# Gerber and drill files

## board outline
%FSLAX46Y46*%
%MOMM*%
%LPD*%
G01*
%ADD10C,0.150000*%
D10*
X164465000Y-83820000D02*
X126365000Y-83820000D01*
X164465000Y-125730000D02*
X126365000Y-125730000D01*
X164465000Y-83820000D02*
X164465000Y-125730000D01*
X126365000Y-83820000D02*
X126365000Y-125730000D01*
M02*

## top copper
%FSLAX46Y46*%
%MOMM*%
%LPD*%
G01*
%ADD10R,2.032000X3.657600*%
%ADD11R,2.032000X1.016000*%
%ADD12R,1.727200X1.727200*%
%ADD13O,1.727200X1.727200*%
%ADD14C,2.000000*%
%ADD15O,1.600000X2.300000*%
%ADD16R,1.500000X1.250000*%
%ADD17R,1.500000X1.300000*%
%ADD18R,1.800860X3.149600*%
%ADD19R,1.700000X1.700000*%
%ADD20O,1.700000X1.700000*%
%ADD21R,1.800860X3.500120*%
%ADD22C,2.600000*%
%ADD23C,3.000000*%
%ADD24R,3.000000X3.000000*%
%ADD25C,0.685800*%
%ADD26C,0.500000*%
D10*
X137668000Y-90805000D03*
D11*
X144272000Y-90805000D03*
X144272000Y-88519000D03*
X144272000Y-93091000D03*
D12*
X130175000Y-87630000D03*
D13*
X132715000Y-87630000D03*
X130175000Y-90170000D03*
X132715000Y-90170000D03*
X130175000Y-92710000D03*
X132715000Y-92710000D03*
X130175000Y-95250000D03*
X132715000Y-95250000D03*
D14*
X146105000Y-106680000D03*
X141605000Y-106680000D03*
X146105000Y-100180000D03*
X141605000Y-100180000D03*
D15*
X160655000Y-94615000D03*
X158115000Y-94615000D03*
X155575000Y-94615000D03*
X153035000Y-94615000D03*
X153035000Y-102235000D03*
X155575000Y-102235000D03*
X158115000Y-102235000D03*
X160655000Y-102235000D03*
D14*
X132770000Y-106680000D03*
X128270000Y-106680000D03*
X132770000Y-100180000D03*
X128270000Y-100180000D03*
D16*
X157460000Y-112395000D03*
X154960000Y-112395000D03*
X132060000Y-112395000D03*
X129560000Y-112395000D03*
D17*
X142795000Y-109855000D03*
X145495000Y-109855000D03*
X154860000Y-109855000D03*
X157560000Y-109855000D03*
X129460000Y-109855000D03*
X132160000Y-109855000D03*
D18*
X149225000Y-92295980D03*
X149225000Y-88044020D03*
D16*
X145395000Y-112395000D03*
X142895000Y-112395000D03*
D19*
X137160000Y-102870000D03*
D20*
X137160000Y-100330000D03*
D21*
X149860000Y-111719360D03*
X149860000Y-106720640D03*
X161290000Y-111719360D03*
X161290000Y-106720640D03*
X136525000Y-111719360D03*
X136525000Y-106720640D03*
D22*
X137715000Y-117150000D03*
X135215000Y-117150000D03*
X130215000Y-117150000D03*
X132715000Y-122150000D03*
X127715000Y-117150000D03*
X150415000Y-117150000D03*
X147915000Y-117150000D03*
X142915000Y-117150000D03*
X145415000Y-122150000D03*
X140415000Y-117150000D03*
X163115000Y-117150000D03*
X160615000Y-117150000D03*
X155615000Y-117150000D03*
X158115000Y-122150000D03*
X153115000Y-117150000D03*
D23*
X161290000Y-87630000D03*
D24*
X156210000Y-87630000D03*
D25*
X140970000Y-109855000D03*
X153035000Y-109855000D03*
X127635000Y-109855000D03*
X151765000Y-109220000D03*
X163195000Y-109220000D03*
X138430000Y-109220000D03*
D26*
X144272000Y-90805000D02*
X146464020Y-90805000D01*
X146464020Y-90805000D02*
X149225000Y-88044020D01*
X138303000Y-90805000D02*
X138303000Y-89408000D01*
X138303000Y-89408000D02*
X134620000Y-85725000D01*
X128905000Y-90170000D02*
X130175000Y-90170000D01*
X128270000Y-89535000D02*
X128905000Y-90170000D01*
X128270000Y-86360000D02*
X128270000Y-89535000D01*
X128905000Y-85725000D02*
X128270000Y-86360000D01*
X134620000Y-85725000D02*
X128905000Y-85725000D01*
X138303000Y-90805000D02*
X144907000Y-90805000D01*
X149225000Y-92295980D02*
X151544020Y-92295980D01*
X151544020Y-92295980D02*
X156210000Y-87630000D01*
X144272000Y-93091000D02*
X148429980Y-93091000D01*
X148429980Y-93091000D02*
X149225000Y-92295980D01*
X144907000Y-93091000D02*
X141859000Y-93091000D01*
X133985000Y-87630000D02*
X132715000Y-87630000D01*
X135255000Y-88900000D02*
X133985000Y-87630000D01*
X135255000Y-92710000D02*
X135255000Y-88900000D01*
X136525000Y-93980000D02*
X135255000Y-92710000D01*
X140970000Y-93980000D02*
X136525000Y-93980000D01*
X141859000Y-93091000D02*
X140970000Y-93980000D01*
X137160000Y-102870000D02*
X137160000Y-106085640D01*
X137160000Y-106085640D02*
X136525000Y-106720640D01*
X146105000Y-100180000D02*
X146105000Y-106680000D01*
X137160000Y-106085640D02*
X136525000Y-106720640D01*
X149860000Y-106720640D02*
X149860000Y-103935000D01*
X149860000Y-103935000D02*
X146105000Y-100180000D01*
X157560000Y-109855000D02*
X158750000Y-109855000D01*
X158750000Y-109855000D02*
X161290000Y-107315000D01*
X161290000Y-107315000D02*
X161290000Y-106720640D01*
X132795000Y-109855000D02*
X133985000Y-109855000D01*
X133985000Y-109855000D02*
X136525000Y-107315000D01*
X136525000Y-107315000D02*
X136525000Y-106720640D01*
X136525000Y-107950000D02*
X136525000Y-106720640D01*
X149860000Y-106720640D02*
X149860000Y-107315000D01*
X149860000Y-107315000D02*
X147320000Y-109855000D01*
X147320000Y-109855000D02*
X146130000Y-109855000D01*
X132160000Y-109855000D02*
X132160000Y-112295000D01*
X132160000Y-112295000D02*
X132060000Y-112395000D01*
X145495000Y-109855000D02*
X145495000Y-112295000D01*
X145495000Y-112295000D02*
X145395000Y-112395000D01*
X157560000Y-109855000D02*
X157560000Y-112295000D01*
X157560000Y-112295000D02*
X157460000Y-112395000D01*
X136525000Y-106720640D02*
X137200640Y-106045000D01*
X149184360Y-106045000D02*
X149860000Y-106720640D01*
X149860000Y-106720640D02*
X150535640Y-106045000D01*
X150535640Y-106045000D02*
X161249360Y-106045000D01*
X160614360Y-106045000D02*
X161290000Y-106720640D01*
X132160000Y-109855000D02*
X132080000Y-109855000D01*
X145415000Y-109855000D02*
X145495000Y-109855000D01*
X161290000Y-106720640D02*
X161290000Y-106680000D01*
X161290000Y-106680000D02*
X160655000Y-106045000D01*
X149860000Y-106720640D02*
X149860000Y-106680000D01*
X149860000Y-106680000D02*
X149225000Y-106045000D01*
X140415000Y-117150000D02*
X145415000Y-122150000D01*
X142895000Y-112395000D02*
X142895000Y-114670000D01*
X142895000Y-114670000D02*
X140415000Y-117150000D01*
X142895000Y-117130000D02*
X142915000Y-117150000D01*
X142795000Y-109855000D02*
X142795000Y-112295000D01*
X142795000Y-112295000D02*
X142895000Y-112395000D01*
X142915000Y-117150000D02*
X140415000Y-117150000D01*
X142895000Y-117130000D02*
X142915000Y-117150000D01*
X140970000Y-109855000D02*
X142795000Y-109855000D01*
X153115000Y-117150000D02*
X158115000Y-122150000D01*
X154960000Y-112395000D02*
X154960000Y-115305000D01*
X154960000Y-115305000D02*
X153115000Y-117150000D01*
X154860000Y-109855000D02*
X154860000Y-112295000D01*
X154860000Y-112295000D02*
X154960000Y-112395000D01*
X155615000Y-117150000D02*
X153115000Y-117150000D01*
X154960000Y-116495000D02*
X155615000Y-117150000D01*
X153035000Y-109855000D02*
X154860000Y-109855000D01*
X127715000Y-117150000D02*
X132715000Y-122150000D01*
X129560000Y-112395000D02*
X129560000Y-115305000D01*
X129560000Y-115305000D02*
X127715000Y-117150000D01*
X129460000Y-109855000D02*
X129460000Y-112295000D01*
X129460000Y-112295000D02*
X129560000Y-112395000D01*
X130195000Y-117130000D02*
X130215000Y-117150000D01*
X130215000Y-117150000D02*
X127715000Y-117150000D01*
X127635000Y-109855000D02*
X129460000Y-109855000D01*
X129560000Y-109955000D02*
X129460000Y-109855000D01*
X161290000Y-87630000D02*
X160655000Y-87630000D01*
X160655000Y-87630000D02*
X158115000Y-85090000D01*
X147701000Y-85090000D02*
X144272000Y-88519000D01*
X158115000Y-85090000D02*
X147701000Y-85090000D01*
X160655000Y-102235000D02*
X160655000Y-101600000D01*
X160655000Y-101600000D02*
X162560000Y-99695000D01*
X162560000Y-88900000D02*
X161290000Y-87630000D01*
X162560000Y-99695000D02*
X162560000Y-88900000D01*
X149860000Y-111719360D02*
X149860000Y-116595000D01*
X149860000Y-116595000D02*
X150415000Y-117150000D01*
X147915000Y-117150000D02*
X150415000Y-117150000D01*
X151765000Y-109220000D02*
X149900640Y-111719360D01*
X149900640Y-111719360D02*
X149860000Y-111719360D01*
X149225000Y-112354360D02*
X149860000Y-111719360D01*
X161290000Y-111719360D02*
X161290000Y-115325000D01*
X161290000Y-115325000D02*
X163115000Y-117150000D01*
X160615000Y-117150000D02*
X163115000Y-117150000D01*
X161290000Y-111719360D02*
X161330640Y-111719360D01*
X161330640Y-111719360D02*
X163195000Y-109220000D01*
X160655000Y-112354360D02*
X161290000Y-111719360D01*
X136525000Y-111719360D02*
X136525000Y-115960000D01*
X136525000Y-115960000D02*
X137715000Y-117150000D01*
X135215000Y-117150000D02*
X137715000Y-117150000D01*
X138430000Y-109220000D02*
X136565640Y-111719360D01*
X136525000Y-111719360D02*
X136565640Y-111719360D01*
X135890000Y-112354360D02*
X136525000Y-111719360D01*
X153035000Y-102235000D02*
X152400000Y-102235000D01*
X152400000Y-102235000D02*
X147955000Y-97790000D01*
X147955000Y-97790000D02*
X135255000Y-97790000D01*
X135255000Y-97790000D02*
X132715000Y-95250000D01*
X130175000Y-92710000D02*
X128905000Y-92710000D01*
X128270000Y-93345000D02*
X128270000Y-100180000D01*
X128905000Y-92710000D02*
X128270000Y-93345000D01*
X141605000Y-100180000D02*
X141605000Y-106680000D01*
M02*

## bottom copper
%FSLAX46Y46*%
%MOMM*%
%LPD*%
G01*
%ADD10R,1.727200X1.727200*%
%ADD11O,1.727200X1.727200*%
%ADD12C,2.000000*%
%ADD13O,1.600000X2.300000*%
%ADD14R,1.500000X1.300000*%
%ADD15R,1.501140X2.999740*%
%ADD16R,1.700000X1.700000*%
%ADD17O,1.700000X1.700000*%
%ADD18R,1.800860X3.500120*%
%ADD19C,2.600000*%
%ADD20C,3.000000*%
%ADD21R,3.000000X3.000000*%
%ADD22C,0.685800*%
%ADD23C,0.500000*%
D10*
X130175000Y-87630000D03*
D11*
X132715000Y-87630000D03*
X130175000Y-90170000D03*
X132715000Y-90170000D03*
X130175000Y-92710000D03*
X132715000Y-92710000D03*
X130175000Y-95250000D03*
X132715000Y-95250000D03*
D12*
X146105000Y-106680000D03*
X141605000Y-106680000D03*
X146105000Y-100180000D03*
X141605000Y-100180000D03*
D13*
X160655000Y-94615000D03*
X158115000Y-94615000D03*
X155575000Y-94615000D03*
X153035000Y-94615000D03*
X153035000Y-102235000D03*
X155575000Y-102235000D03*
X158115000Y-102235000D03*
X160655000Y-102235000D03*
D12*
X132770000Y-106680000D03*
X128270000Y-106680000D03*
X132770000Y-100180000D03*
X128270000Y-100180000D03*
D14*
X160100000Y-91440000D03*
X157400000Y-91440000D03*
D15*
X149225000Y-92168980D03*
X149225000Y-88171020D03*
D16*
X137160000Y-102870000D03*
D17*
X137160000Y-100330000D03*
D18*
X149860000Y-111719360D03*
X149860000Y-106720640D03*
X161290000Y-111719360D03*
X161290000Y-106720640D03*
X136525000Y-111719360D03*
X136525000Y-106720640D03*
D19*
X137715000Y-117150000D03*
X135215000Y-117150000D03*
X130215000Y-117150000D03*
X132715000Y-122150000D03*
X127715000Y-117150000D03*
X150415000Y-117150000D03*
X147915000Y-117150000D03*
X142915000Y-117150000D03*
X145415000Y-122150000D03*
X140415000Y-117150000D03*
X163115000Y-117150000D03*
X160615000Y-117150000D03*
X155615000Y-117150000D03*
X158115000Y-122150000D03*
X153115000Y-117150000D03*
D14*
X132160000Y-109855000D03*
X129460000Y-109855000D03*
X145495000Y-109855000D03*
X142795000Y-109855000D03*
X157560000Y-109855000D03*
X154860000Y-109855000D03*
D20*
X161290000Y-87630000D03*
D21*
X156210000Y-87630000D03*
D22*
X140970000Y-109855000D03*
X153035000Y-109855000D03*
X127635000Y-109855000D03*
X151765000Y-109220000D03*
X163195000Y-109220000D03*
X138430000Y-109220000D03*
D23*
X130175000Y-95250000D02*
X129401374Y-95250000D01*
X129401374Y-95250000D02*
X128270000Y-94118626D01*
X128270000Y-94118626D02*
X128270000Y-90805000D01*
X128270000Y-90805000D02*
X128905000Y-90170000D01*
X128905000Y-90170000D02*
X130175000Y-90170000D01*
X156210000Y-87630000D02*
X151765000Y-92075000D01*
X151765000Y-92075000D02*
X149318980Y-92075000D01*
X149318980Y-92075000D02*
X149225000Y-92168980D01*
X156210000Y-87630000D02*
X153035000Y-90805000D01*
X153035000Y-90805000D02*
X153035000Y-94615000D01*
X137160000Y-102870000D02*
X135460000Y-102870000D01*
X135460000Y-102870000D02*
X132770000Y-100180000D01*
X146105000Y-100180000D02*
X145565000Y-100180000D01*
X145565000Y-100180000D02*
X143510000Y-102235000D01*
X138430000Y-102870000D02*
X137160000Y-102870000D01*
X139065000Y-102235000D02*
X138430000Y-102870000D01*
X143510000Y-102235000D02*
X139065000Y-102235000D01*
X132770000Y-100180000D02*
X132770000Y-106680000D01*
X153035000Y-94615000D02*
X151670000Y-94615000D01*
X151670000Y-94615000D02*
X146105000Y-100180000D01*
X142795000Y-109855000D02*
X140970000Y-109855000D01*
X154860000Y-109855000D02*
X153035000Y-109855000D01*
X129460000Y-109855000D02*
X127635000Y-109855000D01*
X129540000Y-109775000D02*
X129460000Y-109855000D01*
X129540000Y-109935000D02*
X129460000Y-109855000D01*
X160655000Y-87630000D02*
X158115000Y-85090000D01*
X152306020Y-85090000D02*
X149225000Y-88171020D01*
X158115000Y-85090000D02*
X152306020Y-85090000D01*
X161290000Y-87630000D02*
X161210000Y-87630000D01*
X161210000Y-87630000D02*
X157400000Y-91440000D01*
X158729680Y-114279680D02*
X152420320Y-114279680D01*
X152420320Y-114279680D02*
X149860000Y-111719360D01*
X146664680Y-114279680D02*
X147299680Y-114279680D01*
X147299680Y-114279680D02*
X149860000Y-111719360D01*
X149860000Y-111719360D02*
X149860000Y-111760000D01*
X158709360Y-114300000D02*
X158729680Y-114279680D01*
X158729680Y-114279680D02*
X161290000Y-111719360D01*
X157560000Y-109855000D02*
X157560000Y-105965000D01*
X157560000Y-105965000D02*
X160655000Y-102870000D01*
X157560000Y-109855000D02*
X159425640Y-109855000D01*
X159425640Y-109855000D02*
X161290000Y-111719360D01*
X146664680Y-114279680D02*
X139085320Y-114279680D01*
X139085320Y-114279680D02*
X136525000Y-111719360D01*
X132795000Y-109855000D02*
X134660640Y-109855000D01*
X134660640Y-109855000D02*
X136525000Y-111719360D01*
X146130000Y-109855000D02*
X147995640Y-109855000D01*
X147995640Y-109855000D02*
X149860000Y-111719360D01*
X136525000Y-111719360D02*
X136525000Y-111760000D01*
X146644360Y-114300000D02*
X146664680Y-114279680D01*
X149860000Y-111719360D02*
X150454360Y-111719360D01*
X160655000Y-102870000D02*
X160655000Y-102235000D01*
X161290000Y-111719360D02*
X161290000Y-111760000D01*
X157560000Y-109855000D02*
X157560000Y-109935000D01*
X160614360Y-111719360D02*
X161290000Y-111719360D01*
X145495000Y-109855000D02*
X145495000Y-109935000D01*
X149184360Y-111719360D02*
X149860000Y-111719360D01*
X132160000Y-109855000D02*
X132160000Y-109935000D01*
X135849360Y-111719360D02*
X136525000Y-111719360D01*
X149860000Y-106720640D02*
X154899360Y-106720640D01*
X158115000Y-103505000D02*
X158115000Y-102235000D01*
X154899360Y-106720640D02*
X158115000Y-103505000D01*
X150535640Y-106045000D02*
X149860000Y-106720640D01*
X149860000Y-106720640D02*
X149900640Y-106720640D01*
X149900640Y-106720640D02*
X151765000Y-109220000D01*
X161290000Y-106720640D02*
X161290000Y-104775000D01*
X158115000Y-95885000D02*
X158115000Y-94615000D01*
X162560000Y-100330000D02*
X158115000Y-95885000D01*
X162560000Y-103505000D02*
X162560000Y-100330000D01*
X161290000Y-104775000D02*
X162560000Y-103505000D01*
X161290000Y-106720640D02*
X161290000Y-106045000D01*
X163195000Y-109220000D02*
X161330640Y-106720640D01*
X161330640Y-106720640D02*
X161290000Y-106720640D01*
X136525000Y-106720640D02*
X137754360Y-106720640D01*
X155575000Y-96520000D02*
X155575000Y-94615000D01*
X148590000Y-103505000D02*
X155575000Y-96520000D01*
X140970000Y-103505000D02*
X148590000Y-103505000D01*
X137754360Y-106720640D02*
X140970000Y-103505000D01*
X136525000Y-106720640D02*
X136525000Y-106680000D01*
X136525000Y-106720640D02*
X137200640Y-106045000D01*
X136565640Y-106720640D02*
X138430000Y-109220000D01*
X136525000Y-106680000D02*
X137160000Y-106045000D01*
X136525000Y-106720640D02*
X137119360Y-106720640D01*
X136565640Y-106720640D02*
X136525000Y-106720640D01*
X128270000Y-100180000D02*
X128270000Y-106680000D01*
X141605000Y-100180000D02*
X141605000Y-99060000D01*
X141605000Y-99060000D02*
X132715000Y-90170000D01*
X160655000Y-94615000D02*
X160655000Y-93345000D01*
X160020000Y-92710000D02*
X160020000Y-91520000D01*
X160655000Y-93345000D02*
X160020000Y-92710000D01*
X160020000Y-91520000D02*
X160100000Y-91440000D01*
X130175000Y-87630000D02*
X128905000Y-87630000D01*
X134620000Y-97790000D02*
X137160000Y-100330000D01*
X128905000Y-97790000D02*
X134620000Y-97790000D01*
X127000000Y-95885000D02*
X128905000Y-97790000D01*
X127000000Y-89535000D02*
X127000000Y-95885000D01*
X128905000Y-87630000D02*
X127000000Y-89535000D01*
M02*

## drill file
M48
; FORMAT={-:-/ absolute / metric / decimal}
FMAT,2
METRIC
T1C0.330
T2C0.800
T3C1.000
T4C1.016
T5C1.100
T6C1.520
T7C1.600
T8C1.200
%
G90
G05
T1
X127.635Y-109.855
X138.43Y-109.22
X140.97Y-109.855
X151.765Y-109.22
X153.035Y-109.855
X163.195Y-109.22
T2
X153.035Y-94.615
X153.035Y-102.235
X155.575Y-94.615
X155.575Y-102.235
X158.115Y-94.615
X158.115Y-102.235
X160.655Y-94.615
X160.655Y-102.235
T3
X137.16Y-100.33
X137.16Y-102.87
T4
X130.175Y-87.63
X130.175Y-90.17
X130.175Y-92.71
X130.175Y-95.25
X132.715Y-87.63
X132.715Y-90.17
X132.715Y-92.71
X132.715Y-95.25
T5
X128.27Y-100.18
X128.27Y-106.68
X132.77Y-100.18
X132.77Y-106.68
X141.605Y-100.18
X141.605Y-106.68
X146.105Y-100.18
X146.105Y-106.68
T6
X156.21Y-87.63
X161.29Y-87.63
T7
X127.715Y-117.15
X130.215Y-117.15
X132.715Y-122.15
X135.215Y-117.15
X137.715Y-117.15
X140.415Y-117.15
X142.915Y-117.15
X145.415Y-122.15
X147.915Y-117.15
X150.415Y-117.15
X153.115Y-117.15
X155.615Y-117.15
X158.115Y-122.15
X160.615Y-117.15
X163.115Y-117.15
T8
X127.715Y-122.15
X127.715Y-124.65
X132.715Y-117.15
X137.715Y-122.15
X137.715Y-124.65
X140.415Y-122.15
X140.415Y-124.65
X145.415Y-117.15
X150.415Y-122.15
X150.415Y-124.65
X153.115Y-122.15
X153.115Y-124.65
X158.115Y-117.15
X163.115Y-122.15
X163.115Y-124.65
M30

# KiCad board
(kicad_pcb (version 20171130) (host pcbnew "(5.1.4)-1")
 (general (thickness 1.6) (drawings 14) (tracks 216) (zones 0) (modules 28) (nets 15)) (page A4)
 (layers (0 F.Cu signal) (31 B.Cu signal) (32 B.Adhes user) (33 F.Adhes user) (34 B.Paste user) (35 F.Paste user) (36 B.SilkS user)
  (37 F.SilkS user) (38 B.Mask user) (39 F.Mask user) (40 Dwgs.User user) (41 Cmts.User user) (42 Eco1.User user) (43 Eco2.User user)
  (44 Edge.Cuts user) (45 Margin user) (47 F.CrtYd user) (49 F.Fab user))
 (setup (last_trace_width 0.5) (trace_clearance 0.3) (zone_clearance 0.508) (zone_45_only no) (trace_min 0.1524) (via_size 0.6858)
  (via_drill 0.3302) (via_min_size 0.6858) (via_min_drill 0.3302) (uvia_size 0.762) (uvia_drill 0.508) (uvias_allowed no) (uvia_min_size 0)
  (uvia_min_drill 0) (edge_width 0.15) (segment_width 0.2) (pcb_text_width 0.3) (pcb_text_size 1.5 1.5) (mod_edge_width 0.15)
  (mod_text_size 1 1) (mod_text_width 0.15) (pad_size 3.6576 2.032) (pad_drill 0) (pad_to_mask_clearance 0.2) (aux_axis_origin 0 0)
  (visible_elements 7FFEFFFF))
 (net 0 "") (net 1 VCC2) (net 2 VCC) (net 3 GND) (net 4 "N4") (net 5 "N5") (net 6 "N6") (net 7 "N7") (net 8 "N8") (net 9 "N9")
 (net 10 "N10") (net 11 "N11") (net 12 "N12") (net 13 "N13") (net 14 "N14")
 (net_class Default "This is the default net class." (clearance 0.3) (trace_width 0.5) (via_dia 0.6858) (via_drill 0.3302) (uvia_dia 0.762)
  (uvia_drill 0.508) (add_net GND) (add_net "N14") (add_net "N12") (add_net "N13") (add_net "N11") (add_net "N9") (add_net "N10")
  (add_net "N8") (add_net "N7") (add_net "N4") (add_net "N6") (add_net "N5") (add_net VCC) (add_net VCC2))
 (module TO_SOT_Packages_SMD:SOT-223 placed (layer F.Cu) (at 140.97 90.805 90)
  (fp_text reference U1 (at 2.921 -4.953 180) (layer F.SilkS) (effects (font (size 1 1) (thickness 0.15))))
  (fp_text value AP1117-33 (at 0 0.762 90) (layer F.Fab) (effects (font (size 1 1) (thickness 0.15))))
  (pad 2 smd rect (at 0 -3.302 90) (size 3.6576 2.032) (layers F.Cu F.Paste F.Mask) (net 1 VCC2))
  (pad 2 smd rect (at 0 3.302 90) (size 1.016 2.032) (layers F.Cu F.Paste F.Mask) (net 1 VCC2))
  (pad 3 smd rect (at 2.286 3.302 90) (size 1.016 2.032) (layers F.Cu F.Paste F.Mask) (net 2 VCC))
  (pad 1 smd rect (at -2.286 3.302 90) (size 1.016 2.032) (layers F.Cu F.Paste F.Mask) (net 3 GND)))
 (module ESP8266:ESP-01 (layer F.Cu) (at 130.175 87.63)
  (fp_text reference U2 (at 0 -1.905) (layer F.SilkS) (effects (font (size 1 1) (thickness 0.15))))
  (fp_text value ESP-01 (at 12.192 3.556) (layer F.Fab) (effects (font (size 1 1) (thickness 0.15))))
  (pad 1 thru_hole rect (at 0 0) (size 1.7272 1.7272) (drill 1.016) (layers *.Cu *.Mask F.SilkS) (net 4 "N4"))
  (pad 2 thru_hole oval (at 2.54 0) (size 1.7272 1.7272) (drill 1.016) (layers *.Cu *.Mask F.SilkS) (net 3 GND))
  (pad 3 thru_hole oval (at 0 2.54) (size 1.7272 1.7272) (drill 1.016) (layers *.Cu *.Mask F.SilkS) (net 1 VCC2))
  (pad 4 thru_hole oval (at 2.54 2.54) (size 1.7272 1.7272) (drill 1.016) (layers *.Cu *.Mask F.SilkS) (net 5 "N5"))
  (pad 5 thru_hole oval (at 0 5.08) (size 1.7272 1.7272) (drill 1.016) (layers *.Cu *.Mask F.SilkS) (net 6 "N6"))
  (pad 6 thru_hole oval (at 2.54 5.08) (size 1.7272 1.7272) (drill 1.016) (layers *.Cu *.Mask F.SilkS))
  (pad 7 thru_hole oval (at 0 7.62) (size 1.7272 1.7272) (drill 1.016) (layers *.Cu *.Mask F.SilkS) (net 1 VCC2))
  (pad 8 thru_hole oval (at 2.54 7.62) (size 1.7272 1.7272) (drill 1.016) (layers *.Cu *.Mask F.SilkS) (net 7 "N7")))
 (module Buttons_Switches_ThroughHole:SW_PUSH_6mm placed (layer F.Cu) (at 141.605 106.68 90)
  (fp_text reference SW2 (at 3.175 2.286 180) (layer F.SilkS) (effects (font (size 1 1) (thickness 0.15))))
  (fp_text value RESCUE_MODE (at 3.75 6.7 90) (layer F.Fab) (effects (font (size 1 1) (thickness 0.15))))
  (pad 2 thru_hole circle (at 0 4.5 180) (size 2 2) (drill 1.1) (layers *.Cu *.Mask) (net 3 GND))
  (pad 1 thru_hole circle (at 0 0 180) (size 2 2) (drill 1.1) (layers *.Cu *.Mask) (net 5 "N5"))
  (pad 2 thru_hole circle (at 6.5 4.5 180) (size 2 2) (drill 1.1) (layers *.Cu *.Mask) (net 3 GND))
  (pad 1 thru_hole circle (at 6.5 0 180) (size 2 2) (drill 1.1) (layers *.Cu *.Mask) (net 5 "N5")))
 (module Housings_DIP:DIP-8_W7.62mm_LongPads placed (layer F.Cu) (at 160.655 94.615 270)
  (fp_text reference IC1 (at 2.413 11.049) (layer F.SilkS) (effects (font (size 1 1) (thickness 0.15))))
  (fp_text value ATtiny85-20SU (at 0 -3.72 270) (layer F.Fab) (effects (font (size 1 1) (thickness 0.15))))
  (pad 1 thru_hole oval (at 0 0 270) (size 2.3 1.6) (drill 0.8) (layers *.Cu *.Mask F.SilkS) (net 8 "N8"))
  (pad 2 thru_hole oval (at 0 2.54 270) (size 2.3 1.6) (drill 0.8) (layers *.Cu *.Mask F.SilkS) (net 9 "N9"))
  (pad 3 thru_hole oval (at 0 5.08 270) (size 2.3 1.6) (drill 0.8) (layers *.Cu *.Mask F.SilkS) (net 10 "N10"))
  (pad 4 thru_hole oval (at 0 7.62 270) (size 2.3 1.6) (drill 0.8) (layers *.Cu *.Mask F.SilkS) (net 3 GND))
  (pad 5 thru_hole oval (at 7.62 7.62 270) (size 2.3 1.6) (drill 0.8) (layers *.Cu *.Mask F.SilkS) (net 7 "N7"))
  (pad 6 thru_hole oval (at 7.62 5.08 270) (size 2.3 1.6) (drill 0.8) (layers *.Cu *.Mask F.SilkS))
  (pad 7 thru_hole oval (at 7.62 2.54 270) (size 2.3 1.6) (drill 0.8) (layers *.Cu *.Mask F.SilkS) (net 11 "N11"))
  (pad 8 thru_hole oval (at 7.62 0 270) (size 2.3 1.6) (drill 0.8) (layers *.Cu *.Mask F.SilkS) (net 2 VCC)))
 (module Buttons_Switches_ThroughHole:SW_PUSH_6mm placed (layer F.Cu) (at 128.27 106.68 90)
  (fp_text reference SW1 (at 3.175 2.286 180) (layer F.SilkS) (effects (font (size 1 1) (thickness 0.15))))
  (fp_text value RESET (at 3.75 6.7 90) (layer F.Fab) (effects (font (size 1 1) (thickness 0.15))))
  (pad 2 thru_hole circle (at 0 4.5 180) (size 2 2) (drill 1.1) (layers *.Cu *.Mask) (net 3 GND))
  (pad 1 thru_hole circle (at 0 0 180) (size 2 2) (drill 1.1) (layers *.Cu *.Mask) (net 6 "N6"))
  (pad 2 thru_hole circle (at 6.5 4.5 180) (size 2 2) (drill 1.1) (layers *.Cu *.Mask) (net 3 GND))
  (pad 1 thru_hole circle (at 6.5 0 180) (size 2 2) (drill 1.1) (layers *.Cu *.Mask) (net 6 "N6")))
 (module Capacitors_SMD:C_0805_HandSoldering (layer F.Cu) (at 156.21 112.395 180)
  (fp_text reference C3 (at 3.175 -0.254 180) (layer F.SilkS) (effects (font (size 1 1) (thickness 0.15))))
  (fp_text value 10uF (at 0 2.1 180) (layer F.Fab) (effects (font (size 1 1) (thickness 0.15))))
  (pad 1 smd rect (at -1.25 0 180) (size 1.5 1.25) (layers F.Cu F.Paste F.Mask) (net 3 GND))
  (pad 2 smd rect (at 1.25 0 180) (size 1.5 1.25) (layers F.Cu F.Paste F.Mask) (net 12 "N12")))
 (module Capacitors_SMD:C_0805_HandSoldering (layer F.Cu) (at 130.81 112.395 180)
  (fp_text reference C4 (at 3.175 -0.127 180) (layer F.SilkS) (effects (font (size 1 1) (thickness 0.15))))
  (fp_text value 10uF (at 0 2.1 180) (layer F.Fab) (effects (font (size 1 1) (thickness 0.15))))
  (pad 1 smd rect (at -1.25 0 180) (size 1.5 1.25) (layers F.Cu F.Paste F.Mask) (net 3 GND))
  (pad 2 smd rect (at 1.25 0 180) (size 1.5 1.25) (layers F.Cu F.Paste F.Mask) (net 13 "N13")))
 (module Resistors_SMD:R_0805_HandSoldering (layer F.Cu) (at 144.145 109.855)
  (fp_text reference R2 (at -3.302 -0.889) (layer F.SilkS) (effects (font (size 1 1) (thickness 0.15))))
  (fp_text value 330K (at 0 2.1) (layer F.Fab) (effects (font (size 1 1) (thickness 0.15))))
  (pad 1 smd rect (at -1.35 0) (size 1.5 1.3) (layers F.Cu F.Paste F.Mask) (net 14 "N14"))
  (pad 2 smd rect (at 1.35 0) (size 1.5 1.3) (layers F.Cu F.Paste F.Mask) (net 3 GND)))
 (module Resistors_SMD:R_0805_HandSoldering (layer F.Cu) (at 156.21 109.855)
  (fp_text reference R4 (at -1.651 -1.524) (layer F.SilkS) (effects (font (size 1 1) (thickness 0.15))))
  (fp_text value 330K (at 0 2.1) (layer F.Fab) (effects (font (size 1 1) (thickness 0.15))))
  (pad 1 smd rect (at -1.35 0) (size 1.5 1.3) (layers F.Cu F.Paste F.Mask) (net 12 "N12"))
  (pad 2 smd rect (at 1.35 0) (size 1.5 1.3) (layers F.Cu F.Paste F.Mask) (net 3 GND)))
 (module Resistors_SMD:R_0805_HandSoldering (layer F.Cu) (at 130.81 109.855)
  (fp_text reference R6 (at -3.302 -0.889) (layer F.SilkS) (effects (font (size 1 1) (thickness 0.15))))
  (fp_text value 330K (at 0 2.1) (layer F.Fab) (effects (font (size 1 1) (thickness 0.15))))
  (pad 1 smd rect (at -1.35 0) (size 1.5 1.3) (layers F.Cu F.Paste F.Mask) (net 13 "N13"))
  (pad 2 smd rect (at 1.35 0) (size 1.5 1.3) (layers F.Cu F.Paste F.Mask) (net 3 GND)))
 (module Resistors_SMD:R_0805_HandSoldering (layer B.Cu) (at 158.75 91.44 180)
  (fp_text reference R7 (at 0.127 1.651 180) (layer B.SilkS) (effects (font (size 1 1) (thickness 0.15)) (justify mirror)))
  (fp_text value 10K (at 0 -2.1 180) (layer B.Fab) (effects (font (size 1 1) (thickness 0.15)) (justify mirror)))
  (pad 1 smd rect (at -1.35 0 180) (size 1.5 1.3) (layers B.Cu B.Paste B.Mask) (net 8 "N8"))
  (pad 2 smd rect (at 1.35 0 180) (size 1.5 1.3) (layers B.Cu B.Paste B.Mask) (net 2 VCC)))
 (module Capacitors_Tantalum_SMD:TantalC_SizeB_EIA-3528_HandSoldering (layer F.Cu) (at 149.225 90.17 270)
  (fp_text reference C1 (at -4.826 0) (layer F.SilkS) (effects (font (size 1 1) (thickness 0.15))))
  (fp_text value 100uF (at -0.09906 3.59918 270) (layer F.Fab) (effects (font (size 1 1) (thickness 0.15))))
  (pad 2 smd rect (at 2.12598 0 270) (size 3.1496 1.80086) (layers F.Cu F.Paste F.Mask) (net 3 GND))
  (pad 1 smd rect (at -2.12598 0 270) (size 3.1496 1.80086) (layers F.Cu F.Paste F.Mask) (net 1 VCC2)))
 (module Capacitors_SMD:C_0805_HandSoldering (layer F.Cu) (at 144.145 112.395 180)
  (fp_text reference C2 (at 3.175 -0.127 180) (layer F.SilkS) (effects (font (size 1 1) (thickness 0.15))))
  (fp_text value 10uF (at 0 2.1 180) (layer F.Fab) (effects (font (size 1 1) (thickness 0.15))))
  (pad 1 smd rect (at -1.25 0 180) (size 1.5 1.25) (layers F.Cu F.Paste F.Mask) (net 3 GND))
  (pad 2 smd rect (at 1.25 0 180) (size 1.5 1.25) (layers F.Cu F.Paste F.Mask) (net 14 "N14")))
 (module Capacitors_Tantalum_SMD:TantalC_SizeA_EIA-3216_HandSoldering (layer B.Cu) (at 149.225 90.17 270)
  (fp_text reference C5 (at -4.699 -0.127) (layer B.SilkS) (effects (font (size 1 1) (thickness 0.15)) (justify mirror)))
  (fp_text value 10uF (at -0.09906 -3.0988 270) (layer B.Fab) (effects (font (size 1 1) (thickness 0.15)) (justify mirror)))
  (pad 2 smd rect (at 1.99898 0 270) (size 2.99974 1.50114) (layers B.Cu B.Paste B.Mask) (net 3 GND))
  (pad 1 smd rect (at -1.99898 0 270) (size 2.99974 1.50114) (layers B.Cu B.Paste B.Mask) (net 2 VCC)))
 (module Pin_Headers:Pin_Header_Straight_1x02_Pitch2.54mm (layer F.Cu) (at 137.16 102.87 180)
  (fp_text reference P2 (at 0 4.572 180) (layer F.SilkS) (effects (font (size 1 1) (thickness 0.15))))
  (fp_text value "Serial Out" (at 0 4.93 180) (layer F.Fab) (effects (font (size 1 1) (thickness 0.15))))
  (pad 1 thru_hole rect (at 0 0 180) (size 1.7 1.7) (drill 1) (layers *.Cu *.Mask) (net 3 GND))
  (pad 2 thru_hole oval (at 0 2.54 180) (size 1.7 1.7) (drill 1) (layers *.Cu *.Mask) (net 4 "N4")))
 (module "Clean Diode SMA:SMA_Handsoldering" (layer B.Cu) (at 149.86 109.22 90)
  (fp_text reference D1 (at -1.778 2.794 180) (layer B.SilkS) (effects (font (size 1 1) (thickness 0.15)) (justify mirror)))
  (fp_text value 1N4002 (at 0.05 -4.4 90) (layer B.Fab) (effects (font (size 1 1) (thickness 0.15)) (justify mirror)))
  (pad 1 smd rect (at -2.49936 0 90) (size 3.50012 1.80086) (layers B.Cu B.Paste B.Mask) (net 2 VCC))
  (pad 2 smd rect (at 2.49936 0 90) (size 3.50012 1.80086) (layers B.Cu B.Paste B.Mask) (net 11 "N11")))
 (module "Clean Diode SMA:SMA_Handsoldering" (layer F.Cu) (at 149.86 109.22 90)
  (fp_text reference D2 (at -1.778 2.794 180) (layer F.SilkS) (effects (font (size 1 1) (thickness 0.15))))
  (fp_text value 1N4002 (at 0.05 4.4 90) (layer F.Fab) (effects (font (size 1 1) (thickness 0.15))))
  (pad 1 smd rect (at -2.49936 0 90) (size 3.50012 1.80086) (layers F.Cu F.Paste F.Mask) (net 11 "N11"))
  (pad 2 smd rect (at 2.49936 0 90) (size 3.50012 1.80086) (layers F.Cu F.Paste F.Mask) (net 3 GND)))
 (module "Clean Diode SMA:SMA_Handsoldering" (layer B.Cu) (at 161.29 109.22 90)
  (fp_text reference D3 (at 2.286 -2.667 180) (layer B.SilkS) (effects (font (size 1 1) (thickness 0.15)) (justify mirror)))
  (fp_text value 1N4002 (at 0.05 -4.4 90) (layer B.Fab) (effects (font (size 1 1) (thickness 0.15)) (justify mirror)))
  (pad 1 smd rect (at -2.49936 0 90) (size 3.50012 1.80086) (layers B.Cu B.Paste B.Mask) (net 2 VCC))
  (pad 2 smd rect (at 2.49936 0 90) (size 3.50012 1.80086) (layers B.Cu B.Paste B.Mask) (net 9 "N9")))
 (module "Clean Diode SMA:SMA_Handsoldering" (layer F.Cu) (at 161.29 109.22 90)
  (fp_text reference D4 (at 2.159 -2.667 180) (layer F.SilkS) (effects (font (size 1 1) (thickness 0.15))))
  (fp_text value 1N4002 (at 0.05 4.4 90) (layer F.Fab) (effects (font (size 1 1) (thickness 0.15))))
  (pad 1 smd rect (at -2.49936 0 90) (size 3.50012 1.80086) (layers F.Cu F.Paste F.Mask) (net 9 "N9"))
  (pad 2 smd rect (at 2.49936 0 90) (size 3.50012 1.80086) (layers F.Cu F.Paste F.Mask) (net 3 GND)))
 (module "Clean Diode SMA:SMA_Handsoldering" (layer B.Cu) (at 136.525 109.22 90)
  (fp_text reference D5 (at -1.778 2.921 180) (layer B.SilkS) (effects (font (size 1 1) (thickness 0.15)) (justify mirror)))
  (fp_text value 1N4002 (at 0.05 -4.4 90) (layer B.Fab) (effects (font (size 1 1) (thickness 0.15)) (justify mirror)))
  (pad 1 smd rect (at -2.49936 0 90) (size 3.50012 1.80086) (layers B.Cu B.Paste B.Mask) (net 2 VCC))
  (pad 2 smd rect (at 2.49936 0 90) (size 3.50012 1.80086) (layers B.Cu B.Paste B.Mask) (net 10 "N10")))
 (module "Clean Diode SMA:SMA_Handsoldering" (layer F.Cu) (at 136.525 109.22 90)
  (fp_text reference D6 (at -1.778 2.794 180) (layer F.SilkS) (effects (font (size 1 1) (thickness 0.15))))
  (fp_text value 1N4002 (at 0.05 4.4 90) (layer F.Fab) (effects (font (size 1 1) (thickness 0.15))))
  (pad 1 smd rect (at -2.49936 0 90) (size 3.50012 1.80086) (layers F.Cu F.Paste F.Mask) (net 10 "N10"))
  (pad 2 smd rect (at 2.49936 0 90) (size 3.50012 1.80086) (layers F.Cu F.Paste F.Mask) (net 3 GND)))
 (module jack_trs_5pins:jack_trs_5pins (layer F.Cu) (at 132.715 120.65 90)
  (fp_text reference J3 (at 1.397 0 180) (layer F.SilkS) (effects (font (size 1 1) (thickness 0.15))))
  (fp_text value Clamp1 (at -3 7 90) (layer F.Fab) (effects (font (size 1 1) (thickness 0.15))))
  (pad "" np_thru_hole circle (at -4 5 90) (size 1.2 1.2) (drill 1.2) (layers *.Cu *.Mask F.SilkS))
  (pad "" np_thru_hole circle (at -4 -5 90) (size 1.2 1.2) (drill 1.2) (layers *.Cu *.Mask F.SilkS))
  (pad "" np_thru_hole circle (at -1.5 5 90) (size 1.2 1.2) (drill 1.2) (layers *.Cu *.Mask F.SilkS))
  (pad "" np_thru_hole circle (at -1.5 -5 90) (size 1.2 1.2) (drill 1.2) (layers *.Cu *.Mask F.SilkS))
  (pad 5 thru_hole circle (at 3.5 5 180) (size 2.6 2.6) (drill 1.6) (layers *.Cu *.Mask) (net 10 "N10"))
  (pad 4 thru_hole circle (at 3.5 2.5 180) (size 2.6 2.6) (drill 1.6) (layers *.Cu *.Mask) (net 10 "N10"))
  (pad 3 thru_hole circle (at 3.5 -2.5 180) (size 2.6 2.6) (drill 1.6) (layers *.Cu *.Mask) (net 13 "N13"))
  (pad 1 thru_hole circle (at -1.5 0 90) (size 2.6 2.6) (drill 1.6) (layers *.Cu *.Mask) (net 13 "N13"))
  (pad 2 thru_hole circle (at 3.5 -5 180) (size 2.6 2.6) (drill 1.6) (layers *.Cu *.Mask) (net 13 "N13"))
  (pad "" np_thru_hole circle (at 3.5 0 90) (size 1.2 1.2) (drill 1.2) (layers *.Cu *.Mask F.SilkS)))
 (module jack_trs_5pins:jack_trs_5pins (layer F.Cu) (at 145.415 120.65 90)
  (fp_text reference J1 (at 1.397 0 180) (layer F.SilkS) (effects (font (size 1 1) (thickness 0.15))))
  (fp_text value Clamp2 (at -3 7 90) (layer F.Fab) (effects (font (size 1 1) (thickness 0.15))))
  (pad "" np_thru_hole circle (at -4 5 90) (size 1.2 1.2) (drill 1.2) (layers *.Cu *.Mask F.SilkS))
  (pad "" np_thru_hole circle (at -4 -5 90) (size 1.2 1.2) (drill 1.2) (layers *.Cu *.Mask F.SilkS))
  (pad "" np_thru_hole circle (at -1.5 5 90) (size 1.2 1.2) (drill 1.2) (layers *.Cu *.Mask F.SilkS))
  (pad "" np_thru_hole circle (at -1.5 -5 90) (size 1.2 1.2) (drill 1.2) (layers *.Cu *.Mask F.SilkS))
  (pad 5 thru_hole circle (at 3.5 5 180) (size 2.6 2.6) (drill 1.6) (layers *.Cu *.Mask) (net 11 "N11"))
  (pad 4 thru_hole circle (at 3.5 2.5 180) (size 2.6 2.6) (drill 1.6) (layers *.Cu *.Mask) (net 11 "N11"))
  (pad 3 thru_hole circle (at 3.5 -2.5 180) (size 2.6 2.6) (drill 1.6) (layers *.Cu *.Mask) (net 14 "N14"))
  (pad 1 thru_hole circle (at -1.5 0 90) (size 2.6 2.6) (drill 1.6) (layers *.Cu *.Mask) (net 14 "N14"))
  (pad 2 thru_hole circle (at 3.5 -5 180) (size 2.6 2.6) (drill 1.6) (layers *.Cu *.Mask) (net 14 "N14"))
  (pad "" np_thru_hole circle (at 3.5 0 90) (size 1.2 1.2) (drill 1.2) (layers *.Cu *.Mask F.SilkS)))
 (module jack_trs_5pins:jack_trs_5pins (layer F.Cu) (at 158.115 120.65 90)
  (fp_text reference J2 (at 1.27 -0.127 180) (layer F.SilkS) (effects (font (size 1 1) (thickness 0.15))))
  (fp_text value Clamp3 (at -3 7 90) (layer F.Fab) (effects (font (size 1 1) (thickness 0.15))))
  (pad "" np_thru_hole circle (at -4 5 90) (size 1.2 1.2) (drill 1.2) (layers *.Cu *.Mask F.SilkS))
  (pad "" np_thru_hole circle (at -4 -5 90) (size 1.2 1.2) (drill 1.2) (layers *.Cu *.Mask F.SilkS))
  (pad "" np_thru_hole circle (at -1.5 5 90) (size 1.2 1.2) (drill 1.2) (layers *.Cu *.Mask F.SilkS))
  (pad "" np_thru_hole circle (at -1.5 -5 90) (size 1.2 1.2) (drill 1.2) (layers *.Cu *.Mask F.SilkS))
  (pad 5 thru_hole circle (at 3.5 5 180) (size 2.6 2.6) (drill 1.6) (layers *.Cu *.Mask) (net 9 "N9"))
  (pad 4 thru_hole circle (at 3.5 2.5 180) (size 2.6 2.6) (drill 1.6) (layers *.Cu *.Mask) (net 9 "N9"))
  (pad 3 thru_hole circle (at 3.5 -2.5 180) (size 2.6 2.6) (drill 1.6) (layers *.Cu *.Mask) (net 12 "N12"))
  (pad 1 thru_hole circle (at -1.5 0 90) (size 2.6 2.6) (drill 1.6) (layers *.Cu *.Mask) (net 12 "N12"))
  (pad 2 thru_hole circle (at 3.5 -5 180) (size 2.6 2.6) (drill 1.6) (layers *.Cu *.Mask) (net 12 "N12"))
  (pad "" np_thru_hole circle (at 3.5 0 90) (size 1.2 1.2) (drill 1.2) (layers *.Cu *.Mask F.SilkS)))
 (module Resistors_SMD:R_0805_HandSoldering (layer B.Cu) (at 130.81 109.855 180)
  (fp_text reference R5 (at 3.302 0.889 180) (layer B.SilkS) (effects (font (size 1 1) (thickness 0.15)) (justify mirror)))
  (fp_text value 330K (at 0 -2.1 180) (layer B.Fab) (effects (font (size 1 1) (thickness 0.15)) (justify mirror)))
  (pad 1 smd rect (at -1.35 0 180) (size 1.5 1.3) (layers B.Cu B.Paste B.Mask) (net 2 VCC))
  (pad 2 smd rect (at 1.35 0 180) (size 1.5 1.3) (layers B.Cu B.Paste B.Mask) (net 13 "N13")))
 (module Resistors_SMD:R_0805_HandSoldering (layer B.Cu) (at 144.145 109.855 180)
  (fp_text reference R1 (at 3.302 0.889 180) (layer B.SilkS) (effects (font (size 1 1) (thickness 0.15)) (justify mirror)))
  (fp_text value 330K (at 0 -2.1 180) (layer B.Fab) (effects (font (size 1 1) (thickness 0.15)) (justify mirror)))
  (pad 1 smd rect (at -1.35 0 180) (size 1.5 1.3) (layers B.Cu B.Paste B.Mask) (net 2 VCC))
  (pad 2 smd rect (at 1.35 0 180) (size 1.5 1.3) (layers B.Cu B.Paste B.Mask) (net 14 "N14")))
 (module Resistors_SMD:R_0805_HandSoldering (layer B.Cu) (at 156.21 109.855 180)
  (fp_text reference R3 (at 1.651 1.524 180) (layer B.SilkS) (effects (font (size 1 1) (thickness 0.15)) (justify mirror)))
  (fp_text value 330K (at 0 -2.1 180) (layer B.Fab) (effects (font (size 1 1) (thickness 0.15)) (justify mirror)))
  (pad 1 smd rect (at -1.35 0 180) (size 1.5 1.3) (layers B.Cu B.Paste B.Mask) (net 2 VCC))
  (pad 2 smd rect (at 1.35 0 180) (size 1.5 1.3) (layers B.Cu B.Paste B.Mask) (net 12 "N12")))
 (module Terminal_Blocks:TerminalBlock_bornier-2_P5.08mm (layer F.Cu) (at 156.21 87.63)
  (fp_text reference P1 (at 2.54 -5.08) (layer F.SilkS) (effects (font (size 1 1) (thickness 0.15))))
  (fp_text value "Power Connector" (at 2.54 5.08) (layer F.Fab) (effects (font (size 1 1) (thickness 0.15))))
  (pad 2 thru_hole circle (at 5.08 0) (size 3 3) (drill 1.52) (layers *.Cu *.Mask) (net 2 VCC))
  (pad 1 thru_hole rect (at 0 0) (size 3 3) (drill 1.52) (layers *.Cu *.Mask) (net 3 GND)))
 (gr_line (start 164.465 83.82) (end 126.365 83.82) (angle 90) (layer Edge.Cuts) (width 0.15))
 (gr_line (start 164.465 125.73) (end 126.365 125.73) (angle 90) (layer Edge.Cuts) (width 0.15))
 (gr_line (start 164.465 83.82) (end 164.465 125.73) (angle 90) (layer Edge.Cuts) (width 0.15))
 (gr_line (start 126.365 83.82) (end 126.365 125.73) (angle 90) (layer Edge.Cuts) (width 0.15))
 (segment (start 144.272 90.805) (end 146.46402 90.805) (width 0.5) (layer F.Cu) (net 1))
 (segment (start 146.46402 90.805) (end 149.225 88.04402) (width 0.5) (layer F.Cu) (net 1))
 (segment (start 138.303 90.805) (end 138.303 89.408) (width 0.5) (layer F.Cu) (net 1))
 (segment (start 138.303 89.408) (end 134.62 85.725) (width 0.5) (layer F.Cu) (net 1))
 (segment (start 128.905 90.17) (end 130.175 90.17) (width 0.5) (layer F.Cu) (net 1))
 (segment (start 128.27 89.535) (end 128.905 90.17) (width 0.5) (layer F.Cu) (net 1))
 (segment (start 128.27 86.36) (end 128.27 89.535) (width 0.5) (layer F.Cu) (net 1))
 (segment (start 128.905 85.725) (end 128.27 86.36) (width 0.5) (layer F.Cu) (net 1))
 (segment (start 134.62 85.725) (end 128.905 85.725) (width 0.5) (layer F.Cu) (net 1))
 (segment (start 138.303 90.805) (end 144.907 90.805) (width 0.5) (layer F.Cu) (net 1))
 (segment (start 130.175 95.25) (end 129.401374 95.25) (width 0.5) (layer B.Cu) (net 1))
 (segment (start 129.401374 95.25) (end 128.27 94.118626) (width 0.5) (layer B.Cu) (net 1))
 (segment (start 128.27 94.118626) (end 128.27 90.805) (width 0.5) (layer B.Cu) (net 1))
 (segment (start 128.27 90.805) (end 128.905 90.17) (width 0.5) (layer B.Cu) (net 1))
 (segment (start 128.905 90.17) (end 130.175 90.17) (width 0.5) (layer B.Cu) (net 1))
 (segment (start 156.21 87.63) (end 151.765 92.075) (width 0.5) (layer B.Cu) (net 3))
 (segment (start 151.765 92.075) (end 149.31898 92.075) (width 0.5) (layer B.Cu) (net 3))
 (segment (start 149.31898 92.075) (end 149.225 92.16898) (width 0.5) (layer B.Cu) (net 3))
 (segment (start 156.21 87.63) (end 153.035 90.805) (width 0.5) (layer B.Cu) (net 3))
 (segment (start 153.035 90.805) (end 153.035 94.615) (width 0.5) (layer B.Cu) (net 3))
 (segment (start 149.225 92.29598) (end 151.54402 92.29598) (width 0.5) (layer F.Cu) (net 3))
 (segment (start 151.54402 92.29598) (end 156.21 87.63) (width 0.5) (layer F.Cu) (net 3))
 (segment (start 144.272 93.091) (end 148.42998 93.091) (width 0.5) (layer F.Cu) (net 3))
 (segment (start 148.42998 93.091) (end 149.225 92.29598) (width 0.5) (layer F.Cu) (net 3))
 (segment (start 144.907 93.091) (end 141.859 93.091) (width 0.5) (layer F.Cu) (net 3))
 (segment (start 133.985 87.63) (end 132.715 87.63) (width 0.5) (layer F.Cu) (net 3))
 (segment (start 135.255 88.9) (end 133.985 87.63) (width 0.5) (layer F.Cu) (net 3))
 (segment (start 135.255 92.71) (end 135.255 88.9) (width 0.5) (layer F.Cu) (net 3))
 (segment (start 136.525 93.98) (end 135.255 92.71) (width 0.5) (layer F.Cu) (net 3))
 (segment (start 140.97 93.98) (end 136.525 93.98) (width 0.5) (layer F.Cu) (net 3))
 (segment (start 141.859 93.091) (end 140.97 93.98) (width 0.5) (layer F.Cu) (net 3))
 (segment (start 137.16 102.87) (end 137.16 106.08564) (width 0.5) (layer F.Cu) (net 3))
 (segment (start 137.16 106.08564) (end 136.525 106.72064) (width 0.5) (layer F.Cu) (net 3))
 (segment (start 137.16 102.87) (end 135.46 102.87) (width 0.5) (layer B.Cu) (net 3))
 (segment (start 135.46 102.87) (end 132.77 100.18) (width 0.5) (layer B.Cu) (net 3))
 (segment (start 146.105 100.18) (end 145.565 100.18) (width 0.5) (layer B.Cu) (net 3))
 (segment (start 145.565 100.18) (end 143.51 102.235) (width 0.5) (layer B.Cu) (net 3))
 (segment (start 138.43 102.87) (end 137.16 102.87) (width 0.5) (layer B.Cu) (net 3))
 (segment (start 139.065 102.235) (end 138.43 102.87) (width 0.5) (layer B.Cu) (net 3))
 (segment (start 143.51 102.235) (end 139.065 102.235) (width 0.5) (layer B.Cu) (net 3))
 (segment (start 146.105 100.18) (end 146.105 106.68) (width 0.5) (layer F.Cu) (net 3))
 (segment (start 132.77 100.18) (end 132.77 106.68) (width 0.5) (layer B.Cu) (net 3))
 (segment (start 137.16 106.08564) (end 136.525 106.72064) (width 0.5) (layer F.Cu) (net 3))
 (segment (start 149.86 106.72064) (end 149.86 103.935) (width 0.5) (layer F.Cu) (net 3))
 (segment (start 149.86 103.935) (end 146.105 100.18) (width 0.5) (layer F.Cu) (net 3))
 (segment (start 153.035 94.615) (end 151.67 94.615) (width 0.5) (layer B.Cu) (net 3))
 (segment (start 151.67 94.615) (end 146.105 100.18) (width 0.5) (layer B.Cu) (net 3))
 (segment (start 157.56 109.855) (end 158.75 109.855) (width 0.5) (layer F.Cu) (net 3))
 (segment (start 158.75 109.855) (end 161.29 107.315) (width 0.5) (layer F.Cu) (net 3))
 (segment (start 161.29 107.315) (end 161.29 106.72064) (width 0.5) (layer F.Cu) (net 3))
 (segment (start 132.795 109.855) (end 133.985 109.855) (width 0.5) (layer F.Cu) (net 3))
 (segment (start 133.985 109.855) (end 136.525 107.315) (width 0.5) (layer F.Cu) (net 3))
 (segment (start 136.525 107.315) (end 136.525 106.72064) (width 0.5) (layer F.Cu) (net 3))
 (segment (start 136.525 107.95) (end 136.525 106.72064) (width 0.5) (layer F.Cu) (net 3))
 (segment (start 149.86 106.72064) (end 149.86 107.315) (width 0.5) (layer F.Cu) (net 3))
 (segment (start 149.86 107.315) (end 147.32 109.855) (width 0.5) (layer F.Cu) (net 3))
 (segment (start 147.32 109.855) (end 146.13 109.855) (width 0.5) (layer F.Cu) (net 3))
 (segment (start 132.16 109.855) (end 132.16 112.295) (width 0.5) (layer F.Cu) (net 3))
 (segment (start 132.16 112.295) (end 132.06 112.395) (width 0.5) (layer F.Cu) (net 3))
 (segment (start 145.495 109.855) (end 145.495 112.295) (width 0.5) (layer F.Cu) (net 3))
 (segment (start 145.495 112.295) (end 145.395 112.395) (width 0.5) (layer F.Cu) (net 3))
 (segment (start 157.56 109.855) (end 157.56 112.295) (width 0.5) (layer F.Cu) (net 3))
 (segment (start 157.56 112.295) (end 157.46 112.395) (width 0.5) (layer F.Cu) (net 3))
 (segment (start 136.525 106.72064) (end 137.20064 106.045) (width 0.5) (layer F.Cu) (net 3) (status 30))
 (segment (start 149.18436 106.045) (end 149.86 106.72064) (width 0.5) (layer F.Cu) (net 3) (status 30))
 (segment (start 149.86 106.72064) (end 150.53564 106.045) (width 0.5) (layer F.Cu) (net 3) (status 30))
 (segment (start 150.53564 106.045) (end 161.24936 106.045) (width 0.5) (layer F.Cu) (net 3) (status 30))
 (segment (start 160.61436 106.045) (end 161.29 106.72064) (width 0.5) (layer F.Cu) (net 3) (status 30))
 (segment (start 132.16 109.855) (end 132.08 109.855) (width 0.5) (layer F.Cu) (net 3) (status 80030))
 (segment (start 145.415 109.855) (end 145.495 109.855) (width 0.5) (layer F.Cu) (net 3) (status 80030))
 (segment (start 161.29 106.72064) (end 161.29 106.68) (width 0.5) (layer F.Cu) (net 3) (status 30))
 (segment (start 161.29 106.68) (end 160.655 106.045) (width 0.5) (layer F.Cu) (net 3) (status 30))
 (segment (start 149.86 106.72064) (end 149.86 106.68) (width 0.5) (layer F.Cu) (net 3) (status 30))
 (segment (start 149.86 106.68) (end 149.225 106.045) (width 0.5) (layer F.Cu) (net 3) (status 30))
 (segment (start 140.415 117.15) (end 145.415 122.15) (width 0.5) (layer F.Cu) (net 14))
 (segment (start 142.895 112.395) (end 142.895 114.67) (width 0.5) (layer F.Cu) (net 14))
 (segment (start 142.895 114.67) (end 140.415 117.15) (width 0.5) (layer F.Cu) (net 14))
 (segment (start 142.895 117.13) (end 142.915 117.15) (width 0.5) (layer F.Cu) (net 14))
 (segment (start 142.795 109.855) (end 142.795 112.295) (width 0.5) (layer F.Cu) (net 14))
 (segment (start 142.795 112.295) (end 142.895 112.395) (width 0.5) (layer F.Cu) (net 14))
 (segment (start 142.915 117.15) (end 140.415 117.15) (width 0.5) (layer F.Cu) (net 14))
 (segment (start 142.895 117.13) (end 142.915 117.15) (width 0.5) (layer F.Cu) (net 14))
 (segment (start 142.795 109.855) (end 140.97 109.855) (width 0.5) (layer B.Cu) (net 14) (status 10))
 (segment (start 140.97 109.855) (end 142.795 109.855) (width 0.5) (layer F.Cu) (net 14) (status 20))
 (via (at 140.97 109.855) (size 0.6858) (drill 0.3302) (layers F.Cu B.Cu) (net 14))
 (segment (start 153.115 117.15) (end 158.115 122.15) (width 0.5) (layer F.Cu) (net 12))
 (segment (start 154.96 112.395) (end 154.96 115.305) (width 0.5) (layer F.Cu) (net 12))
 (segment (start 154.96 115.305) (end 153.115 117.15) (width 0.5) (layer F.Cu) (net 12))
 (segment (start 154.86 109.855) (end 154.86 112.295) (width 0.5) (layer F.Cu) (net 12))
 (segment (start 154.86 112.295) (end 154.96 112.395) (width 0.5) (layer F.Cu) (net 12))
 (segment (start 155.615 117.15) (end 153.115 117.15) (width 0.5) (layer F.Cu) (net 12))
 (segment (start 154.96 116.495) (end 155.615 117.15) (width 0.5) (layer F.Cu) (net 12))
 (segment (start 154.86 109.855) (end 153.035 109.855) (width 0.5) (layer B.Cu) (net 12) (status 10))
 (segment (start 153.035 109.855) (end 154.86 109.855) (width 0.5) (layer F.Cu) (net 12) (status 20))
 (via (at 153.035 109.855) (size 0.6858) (drill 0.3302) (layers F.Cu B.Cu) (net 12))
 (segment (start 127.715 117.15) (end 132.715 122.15) (width 0.5) (layer F.Cu) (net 13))
 (segment (start 129.56 112.395) (end 129.56 115.305) (width 0.5) (layer F.Cu) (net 13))
 (segment (start 129.56 115.305) (end 127.715 117.15) (width 0.5) (layer F.Cu) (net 13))
 (segment (start 129.46 109.855) (end 129.46 112.295) (width 0.5) (layer F.Cu) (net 13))
 (segment (start 129.46 112.295) (end 129.56 112.395) (width 0.5) (layer F.Cu) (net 13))
 (segment (start 130.195 117.13) (end 130.215 117.15) (width 0.5) (layer F.Cu) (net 13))
 (segment (start 130.215 117.15) (end 127.715 117.15) (width 0.5) (layer F.Cu) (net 13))
 (segment (start 129.46 109.855) (end 127.635 109.855) (width 0.5) (layer B.Cu) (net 13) (status 10))
 (segment (start 127.635 109.855) (end 129.46 109.855) (width 0.5) (layer F.Cu) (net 13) (status 20))
 (via (at 127.635 109.855) (size 0.6858) (drill 0.3302) (layers F.Cu B.Cu) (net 13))
 (segment (start 129.54 109.775) (end 129.46 109.855) (width 0.5) (layer B.Cu) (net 13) (status 30))
 (segment (start 129.54 109.935) (end 129.46 109.855) (width 0.5) (layer B.Cu) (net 13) (status 30))
 (segment (start 129.56 109.955) (end 129.46 109.855) (width 0.5) (layer F.Cu) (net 13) (status 30))
 (segment (start 161.29 87.63) (end 160.655 87.63) (width 0.5) (layer F.Cu) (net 2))
 (segment (start 160.655 87.63) (end 158.115 85.09) (width 0.5) (layer F.Cu) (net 2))
 (segment (start 147.701 85.09) (end 144.272 88.519) (width 0.5) (layer F.Cu) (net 2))
 (segment (start 158.115 85.09) (end 147.701 85.09) (width 0.5) (layer F.Cu) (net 2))
 (segment (start 160.655 87.63) (end 158.115 85.09) (width 0.5) (layer B.Cu) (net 2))
 (segment (start 152.30602 85.09) (end 149.225 88.17102) (width 0.5) (layer B.Cu) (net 2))
 (segment (start 158.115 85.09) (end 152.30602 85.09) (width 0.5) (layer B.Cu) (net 2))
 (segment (start 161.29 87.63) (end 161.21 87.63) (width 0.5) (layer B.Cu) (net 2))
 (segment (start 161.21 87.63) (end 157.4 91.44) (width 0.5) (layer B.Cu) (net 2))
 (segment (start 160.655 102.235) (end 160.655 101.6) (width 0.5) (layer F.Cu) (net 2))
 (segment (start 160.655 101.6) (end 162.56 99.695) (width 0.5) (layer F.Cu) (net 2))
 (segment (start 162.56 88.9) (end 161.29 87.63) (width 0.5) (layer F.Cu) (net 2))
 (segment (start 162.56 99.695) (end 162.56 88.9) (width 0.5) (layer F.Cu) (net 2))
 (segment (start 158.72968 114.27968) (end 152.42032 114.27968) (width 0.5) (layer B.Cu) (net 2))
 (segment (start 152.42032 114.27968) (end 149.86 111.71936) (width 0.5) (layer B.Cu) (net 2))
 (segment (start 146.66468 114.27968) (end 147.29968 114.27968) (width 0.5) (layer B.Cu) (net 2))
 (segment (start 147.29968 114.27968) (end 149.86 111.71936) (width 0.5) (layer B.Cu) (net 2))
 (segment (start 149.86 111.71936) (end 149.86 111.76) (width 0.5) (layer B.Cu) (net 2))
 (segment (start 158.70936 114.3) (end 158.72968 114.27968) (width 0.5) (layer B.Cu) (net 2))
 (segment (start 158.72968 114.27968) (end 161.29 111.71936) (width 0.5) (layer B.Cu) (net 2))
 (segment (start 157.56 109.855) (end 157.56 105.965) (width 0.5) (layer B.Cu) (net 2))
 (segment (start 157.56 105.965) (end 160.655 102.87) (width 0.5) (layer B.Cu) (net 2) (status 20))
 (segment (start 157.56 109.855) (end 159.42564 109.855) (width 0.5) (layer B.Cu) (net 2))
 (segment (start 159.42564 109.855) (end 161.29 111.71936) (width 0.5) (layer B.Cu) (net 2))
 (segment (start 146.66468 114.27968) (end 139.08532 114.27968) (width 0.5) (layer B.Cu) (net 2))
 (segment (start 139.08532 114.27968) (end 136.525 111.71936) (width 0.5) (layer B.Cu) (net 2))
 (segment (start 132.795 109.855) (end 134.66064 109.855) (width 0.5) (layer B.Cu) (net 2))
 (segment (start 134.66064 109.855) (end 136.525 111.71936) (width 0.5) (layer B.Cu) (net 2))
 (segment (start 146.13 109.855) (end 147.99564 109.855) (width 0.5) (layer B.Cu) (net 2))
 (segment (start 147.99564 109.855) (end 149.86 111.71936) (width 0.5) (layer B.Cu) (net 2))
 (segment (start 136.525 111.71936) (end 136.525 111.76) (width 0.5) (layer B.Cu) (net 2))
 (segment (start 146.64436 114.3) (end 146.66468 114.27968) (width 0.5) (layer B.Cu) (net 2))
 (segment (start 149.86 111.71936) (end 150.45436 111.71936) (width 0.5) (layer B.Cu) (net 2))
 (segment (start 160.655 102.87) (end 160.655 102.235) (width 0.5) (layer B.Cu) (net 2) (status 30))
 (segment (start 161.29 111.71936) (end 161.29 111.76) (width 0.5) (layer B.Cu) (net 2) (status 30))
 (segment (start 157.56 109.855) (end 157.56 109.935) (width 0.5) (layer B.Cu) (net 2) (status 30))
 (segment (start 160.61436 111.71936) (end 161.29 111.71936) (width 0.5) (layer B.Cu) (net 2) (status 30))
 (segment (start 145.495 109.855) (end 145.495 109.935) (width 0.5) (layer B.Cu) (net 2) (status 30))
 (segment (start 149.18436 111.71936) (end 149.86 111.71936) (width 0.5) (layer B.Cu) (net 2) (status 30))
 (segment (start 132.16 109.855) (end 132.16 109.935) (width 0.5) (layer B.Cu) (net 2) (status 30))
 (segment (start 135.84936 111.71936) (end 136.525 111.71936) (width 0.5) (layer B.Cu) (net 2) (status 30))
 (segment (start 149.86 106.72064) (end 154.89936 106.72064) (width 0.5) (layer B.Cu) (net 11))
 (segment (start 158.115 103.505) (end 158.115 102.235) (width 0.5) (layer B.Cu) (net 11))
 (segment (start 154.89936 106.72064) (end 158.115 103.505) (width 0.5) (layer B.Cu) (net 11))
 (segment (start 149.86 111.71936) (end 149.86 116.595) (width 0.5) (layer F.Cu) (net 11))
 (segment (start 149.86 116.595) (end 150.415 117.15) (width 0.5) (layer F.Cu) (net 11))
 (segment (start 147.915 117.15) (end 150.415 117.15) (width 0.5) (layer F.Cu) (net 11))
 (segment (start 150.53564 106.045) (end 149.86 106.72064) (width 0.5) (layer B.Cu) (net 11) (status 30))
 (segment (start 149.86 106.72064) (end 149.90064 106.72064) (width 0.5) (layer B.Cu) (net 11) (status 30))
 (segment (start 149.90064 106.72064) (end 151.765 109.22) (width 0.5) (layer B.Cu) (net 11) (status 10))
 (via (at 151.765 109.22) (size 0.6858) (drill 0.3302) (layers F.Cu B.Cu) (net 11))
 (segment (start 151.765 109.22) (end 149.90064 111.71936) (width 0.5) (layer F.Cu) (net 11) (status 20))
 (segment (start 149.90064 111.71936) (end 149.86 111.71936) (width 0.5) (layer F.Cu) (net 11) (status 30))
 (segment (start 149.225 112.35436) (end 149.86 111.71936) (width 0.5) (layer F.Cu) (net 11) (status 30))
 (segment (start 161.29 111.71936) (end 161.29 115.325) (width 0.5) (layer F.Cu) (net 9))
 (segment (start 161.29 115.325) (end 163.115 117.15) (width 0.5) (layer F.Cu) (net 9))
 (segment (start 160.615 117.15) (end 163.115 117.15) (width 0.5) (layer F.Cu) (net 9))
 (segment (start 161.29 106.72064) (end 161.29 104.775) (width 0.5) (layer B.Cu) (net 9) (status 10))
 (segment (start 158.115 95.885) (end 158.115 94.615) (width 0.5) (layer B.Cu) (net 9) (status 20))
 (segment (start 162.56 100.33) (end 158.115 95.885) (width 0.5) (layer B.Cu) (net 9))
 (segment (start 162.56 103.505) (end 162.56 100.33) (width 0.5) (layer B.Cu) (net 9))
 (segment (start 161.29 104.775) (end 162.56 103.505) (width 0.5) (layer B.Cu) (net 9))
 (segment (start 161.29 106.72064) (end 161.29 106.045) (width 0.5) (layer B.Cu) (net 9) (status 30))
 (segment (start 161.29 111.71936) (end 161.33064 111.71936) (width 0.5) (layer F.Cu) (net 9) (status 30))
 (segment (start 161.33064 111.71936) (end 163.195 109.22) (width 0.5) (layer F.Cu) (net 9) (status 10))
 (segment (start 163.195 109.22) (end 161.33064 106.72064) (width 0.5) (layer B.Cu) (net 9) (status 20))
 (via (at 163.195 109.22) (size 0.6858) (drill 0.3302) (layers F.Cu B.Cu) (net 9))
 (segment (start 161.33064 106.72064) (end 161.29 106.72064) (width 0.5) (layer B.Cu) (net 9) (status 30))
 (segment (start 160.655 112.35436) (end 161.29 111.71936) (width 0.5) (layer F.Cu) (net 9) (status 30))
 (segment (start 136.525 111.71936) (end 136.525 115.96) (width 0.5) (layer F.Cu) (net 10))
 (segment (start 136.525 115.96) (end 137.715 117.15) (width 0.5) (layer F.Cu) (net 10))
 (segment (start 136.525 106.72064) (end 137.75436 106.72064) (width 0.5) (layer B.Cu) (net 10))
 (segment (start 155.575 96.52) (end 155.575 94.615) (width 0.5) (layer B.Cu) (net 10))
 (segment (start 148.59 103.505) (end 155.575 96.52) (width 0.5) (layer B.Cu) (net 10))
 (segment (start 140.97 103.505) (end 148.59 103.505) (width 0.5) (layer B.Cu) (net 10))
 (segment (start 137.75436 106.72064) (end 140.97 103.505) (width 0.5) (layer B.Cu) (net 10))
 (segment (start 136.525 106.72064) (end 136.525 106.68) (width 0.5) (layer B.Cu) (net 10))
 (segment (start 135.215 117.15) (end 137.715 117.15) (width 0.5) (layer F.Cu) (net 10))
 (segment (start 136.525 106.72064) (end 137.20064 106.045) (width 0.5) (layer B.Cu) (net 10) (status 30))
 (via (at 138.43 109.22) (size 0.6858) (drill 0.3302) (layers F.Cu B.Cu) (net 10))
 (segment (start 136.56564 106.72064) (end 138.43 109.22) (width 0.5) (layer B.Cu) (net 10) (status 10))
 (segment (start 138.43 109.22) (end 136.56564 111.71936) (width 0.5) (layer F.Cu) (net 10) (status 20))
 (segment (start 136.525 106.68) (end 137.16 106.045) (width 0.5) (layer B.Cu) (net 10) (status 30))
 (segment (start 136.525 106.72064) (end 137.11936 106.72064) (width 0.5) (layer B.Cu) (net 10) (status 30))
 (segment (start 136.525 111.71936) (end 136.56564 111.71936) (width 0.5) (layer F.Cu) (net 10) (status 30))
 (segment (start 136.56564 106.72064) (end 136.525 106.72064) (width 0.5) (layer B.Cu) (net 10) (status 30))
 (segment (start 135.89 112.35436) (end 136.525 111.71936) (width 0.5) (layer F.Cu) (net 10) (status 30))
 (segment (start 153.035 102.235) (end 152.4 102.235) (width 0.5) (layer F.Cu) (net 7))
 (segment (start 152.4 102.235) (end 147.955 97.79) (width 0.5) (layer F.Cu) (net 7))
 (segment (start 147.955 97.79) (end 135.255 97.79) (width 0.5) (layer F.Cu) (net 7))
 (segment (start 135.255 97.79) (end 132.715 95.25) (width 0.5) (layer F.Cu) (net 7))
 (segment (start 130.175 92.71) (end 128.905 92.71) (width 0.5) (layer F.Cu) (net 6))
 (segment (start 128.27 93.345) (end 128.27 100.18) (width 0.5) (layer F.Cu) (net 6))
 (segment (start 128.905 92.71) (end 128.27 93.345) (width 0.5) (layer F.Cu) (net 6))
 (segment (start 128.27 100.18) (end 128.27 106.68) (width 0.5) (layer B.Cu) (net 6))
 (segment (start 141.605 100.18) (end 141.605 99.06) (width 0.5) (layer B.Cu) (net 5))
 (segment (start 141.605 99.06) (end 132.715 90.17) (width 0.5) (layer B.Cu) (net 5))
 (segment (start 141.605 100.18) (end 141.605 106.68) (width 0.5) (layer F.Cu) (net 5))
 (segment (start 160.655 94.615) (end 160.655 93.345) (width 0.5) (layer B.Cu) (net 8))
 (segment (start 160.02 92.71) (end 160.02 91.52) (width 0.5) (layer B.Cu) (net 8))
 (segment (start 160.655 93.345) (end 160.02 92.71) (width 0.5) (layer B.Cu) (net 8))
 (segment (start 160.02 91.52) (end 160.1 91.44) (width 0.5) (layer B.Cu) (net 8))
 (segment (start 130.175 87.63) (end 128.905 87.63) (width 0.5) (layer B.Cu) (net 4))
 (segment (start 134.62 97.79) (end 137.16 100.33) (width 0.5) (layer B.Cu) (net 4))
 (segment (start 128.905 97.79) (end 134.62 97.79) (width 0.5) (layer B.Cu) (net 4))
 (segment (start 127 95.885) (end 128.905 97.79) (width 0.5) (layer B.Cu) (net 4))
 (segment (start 127 89.535) (end 127 95.885) (width 0.5) (layer B.Cu) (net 4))
 (segment (start 128.905 87.63) (end 127 89.535) (width 0.5) (layer B.Cu) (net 4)))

